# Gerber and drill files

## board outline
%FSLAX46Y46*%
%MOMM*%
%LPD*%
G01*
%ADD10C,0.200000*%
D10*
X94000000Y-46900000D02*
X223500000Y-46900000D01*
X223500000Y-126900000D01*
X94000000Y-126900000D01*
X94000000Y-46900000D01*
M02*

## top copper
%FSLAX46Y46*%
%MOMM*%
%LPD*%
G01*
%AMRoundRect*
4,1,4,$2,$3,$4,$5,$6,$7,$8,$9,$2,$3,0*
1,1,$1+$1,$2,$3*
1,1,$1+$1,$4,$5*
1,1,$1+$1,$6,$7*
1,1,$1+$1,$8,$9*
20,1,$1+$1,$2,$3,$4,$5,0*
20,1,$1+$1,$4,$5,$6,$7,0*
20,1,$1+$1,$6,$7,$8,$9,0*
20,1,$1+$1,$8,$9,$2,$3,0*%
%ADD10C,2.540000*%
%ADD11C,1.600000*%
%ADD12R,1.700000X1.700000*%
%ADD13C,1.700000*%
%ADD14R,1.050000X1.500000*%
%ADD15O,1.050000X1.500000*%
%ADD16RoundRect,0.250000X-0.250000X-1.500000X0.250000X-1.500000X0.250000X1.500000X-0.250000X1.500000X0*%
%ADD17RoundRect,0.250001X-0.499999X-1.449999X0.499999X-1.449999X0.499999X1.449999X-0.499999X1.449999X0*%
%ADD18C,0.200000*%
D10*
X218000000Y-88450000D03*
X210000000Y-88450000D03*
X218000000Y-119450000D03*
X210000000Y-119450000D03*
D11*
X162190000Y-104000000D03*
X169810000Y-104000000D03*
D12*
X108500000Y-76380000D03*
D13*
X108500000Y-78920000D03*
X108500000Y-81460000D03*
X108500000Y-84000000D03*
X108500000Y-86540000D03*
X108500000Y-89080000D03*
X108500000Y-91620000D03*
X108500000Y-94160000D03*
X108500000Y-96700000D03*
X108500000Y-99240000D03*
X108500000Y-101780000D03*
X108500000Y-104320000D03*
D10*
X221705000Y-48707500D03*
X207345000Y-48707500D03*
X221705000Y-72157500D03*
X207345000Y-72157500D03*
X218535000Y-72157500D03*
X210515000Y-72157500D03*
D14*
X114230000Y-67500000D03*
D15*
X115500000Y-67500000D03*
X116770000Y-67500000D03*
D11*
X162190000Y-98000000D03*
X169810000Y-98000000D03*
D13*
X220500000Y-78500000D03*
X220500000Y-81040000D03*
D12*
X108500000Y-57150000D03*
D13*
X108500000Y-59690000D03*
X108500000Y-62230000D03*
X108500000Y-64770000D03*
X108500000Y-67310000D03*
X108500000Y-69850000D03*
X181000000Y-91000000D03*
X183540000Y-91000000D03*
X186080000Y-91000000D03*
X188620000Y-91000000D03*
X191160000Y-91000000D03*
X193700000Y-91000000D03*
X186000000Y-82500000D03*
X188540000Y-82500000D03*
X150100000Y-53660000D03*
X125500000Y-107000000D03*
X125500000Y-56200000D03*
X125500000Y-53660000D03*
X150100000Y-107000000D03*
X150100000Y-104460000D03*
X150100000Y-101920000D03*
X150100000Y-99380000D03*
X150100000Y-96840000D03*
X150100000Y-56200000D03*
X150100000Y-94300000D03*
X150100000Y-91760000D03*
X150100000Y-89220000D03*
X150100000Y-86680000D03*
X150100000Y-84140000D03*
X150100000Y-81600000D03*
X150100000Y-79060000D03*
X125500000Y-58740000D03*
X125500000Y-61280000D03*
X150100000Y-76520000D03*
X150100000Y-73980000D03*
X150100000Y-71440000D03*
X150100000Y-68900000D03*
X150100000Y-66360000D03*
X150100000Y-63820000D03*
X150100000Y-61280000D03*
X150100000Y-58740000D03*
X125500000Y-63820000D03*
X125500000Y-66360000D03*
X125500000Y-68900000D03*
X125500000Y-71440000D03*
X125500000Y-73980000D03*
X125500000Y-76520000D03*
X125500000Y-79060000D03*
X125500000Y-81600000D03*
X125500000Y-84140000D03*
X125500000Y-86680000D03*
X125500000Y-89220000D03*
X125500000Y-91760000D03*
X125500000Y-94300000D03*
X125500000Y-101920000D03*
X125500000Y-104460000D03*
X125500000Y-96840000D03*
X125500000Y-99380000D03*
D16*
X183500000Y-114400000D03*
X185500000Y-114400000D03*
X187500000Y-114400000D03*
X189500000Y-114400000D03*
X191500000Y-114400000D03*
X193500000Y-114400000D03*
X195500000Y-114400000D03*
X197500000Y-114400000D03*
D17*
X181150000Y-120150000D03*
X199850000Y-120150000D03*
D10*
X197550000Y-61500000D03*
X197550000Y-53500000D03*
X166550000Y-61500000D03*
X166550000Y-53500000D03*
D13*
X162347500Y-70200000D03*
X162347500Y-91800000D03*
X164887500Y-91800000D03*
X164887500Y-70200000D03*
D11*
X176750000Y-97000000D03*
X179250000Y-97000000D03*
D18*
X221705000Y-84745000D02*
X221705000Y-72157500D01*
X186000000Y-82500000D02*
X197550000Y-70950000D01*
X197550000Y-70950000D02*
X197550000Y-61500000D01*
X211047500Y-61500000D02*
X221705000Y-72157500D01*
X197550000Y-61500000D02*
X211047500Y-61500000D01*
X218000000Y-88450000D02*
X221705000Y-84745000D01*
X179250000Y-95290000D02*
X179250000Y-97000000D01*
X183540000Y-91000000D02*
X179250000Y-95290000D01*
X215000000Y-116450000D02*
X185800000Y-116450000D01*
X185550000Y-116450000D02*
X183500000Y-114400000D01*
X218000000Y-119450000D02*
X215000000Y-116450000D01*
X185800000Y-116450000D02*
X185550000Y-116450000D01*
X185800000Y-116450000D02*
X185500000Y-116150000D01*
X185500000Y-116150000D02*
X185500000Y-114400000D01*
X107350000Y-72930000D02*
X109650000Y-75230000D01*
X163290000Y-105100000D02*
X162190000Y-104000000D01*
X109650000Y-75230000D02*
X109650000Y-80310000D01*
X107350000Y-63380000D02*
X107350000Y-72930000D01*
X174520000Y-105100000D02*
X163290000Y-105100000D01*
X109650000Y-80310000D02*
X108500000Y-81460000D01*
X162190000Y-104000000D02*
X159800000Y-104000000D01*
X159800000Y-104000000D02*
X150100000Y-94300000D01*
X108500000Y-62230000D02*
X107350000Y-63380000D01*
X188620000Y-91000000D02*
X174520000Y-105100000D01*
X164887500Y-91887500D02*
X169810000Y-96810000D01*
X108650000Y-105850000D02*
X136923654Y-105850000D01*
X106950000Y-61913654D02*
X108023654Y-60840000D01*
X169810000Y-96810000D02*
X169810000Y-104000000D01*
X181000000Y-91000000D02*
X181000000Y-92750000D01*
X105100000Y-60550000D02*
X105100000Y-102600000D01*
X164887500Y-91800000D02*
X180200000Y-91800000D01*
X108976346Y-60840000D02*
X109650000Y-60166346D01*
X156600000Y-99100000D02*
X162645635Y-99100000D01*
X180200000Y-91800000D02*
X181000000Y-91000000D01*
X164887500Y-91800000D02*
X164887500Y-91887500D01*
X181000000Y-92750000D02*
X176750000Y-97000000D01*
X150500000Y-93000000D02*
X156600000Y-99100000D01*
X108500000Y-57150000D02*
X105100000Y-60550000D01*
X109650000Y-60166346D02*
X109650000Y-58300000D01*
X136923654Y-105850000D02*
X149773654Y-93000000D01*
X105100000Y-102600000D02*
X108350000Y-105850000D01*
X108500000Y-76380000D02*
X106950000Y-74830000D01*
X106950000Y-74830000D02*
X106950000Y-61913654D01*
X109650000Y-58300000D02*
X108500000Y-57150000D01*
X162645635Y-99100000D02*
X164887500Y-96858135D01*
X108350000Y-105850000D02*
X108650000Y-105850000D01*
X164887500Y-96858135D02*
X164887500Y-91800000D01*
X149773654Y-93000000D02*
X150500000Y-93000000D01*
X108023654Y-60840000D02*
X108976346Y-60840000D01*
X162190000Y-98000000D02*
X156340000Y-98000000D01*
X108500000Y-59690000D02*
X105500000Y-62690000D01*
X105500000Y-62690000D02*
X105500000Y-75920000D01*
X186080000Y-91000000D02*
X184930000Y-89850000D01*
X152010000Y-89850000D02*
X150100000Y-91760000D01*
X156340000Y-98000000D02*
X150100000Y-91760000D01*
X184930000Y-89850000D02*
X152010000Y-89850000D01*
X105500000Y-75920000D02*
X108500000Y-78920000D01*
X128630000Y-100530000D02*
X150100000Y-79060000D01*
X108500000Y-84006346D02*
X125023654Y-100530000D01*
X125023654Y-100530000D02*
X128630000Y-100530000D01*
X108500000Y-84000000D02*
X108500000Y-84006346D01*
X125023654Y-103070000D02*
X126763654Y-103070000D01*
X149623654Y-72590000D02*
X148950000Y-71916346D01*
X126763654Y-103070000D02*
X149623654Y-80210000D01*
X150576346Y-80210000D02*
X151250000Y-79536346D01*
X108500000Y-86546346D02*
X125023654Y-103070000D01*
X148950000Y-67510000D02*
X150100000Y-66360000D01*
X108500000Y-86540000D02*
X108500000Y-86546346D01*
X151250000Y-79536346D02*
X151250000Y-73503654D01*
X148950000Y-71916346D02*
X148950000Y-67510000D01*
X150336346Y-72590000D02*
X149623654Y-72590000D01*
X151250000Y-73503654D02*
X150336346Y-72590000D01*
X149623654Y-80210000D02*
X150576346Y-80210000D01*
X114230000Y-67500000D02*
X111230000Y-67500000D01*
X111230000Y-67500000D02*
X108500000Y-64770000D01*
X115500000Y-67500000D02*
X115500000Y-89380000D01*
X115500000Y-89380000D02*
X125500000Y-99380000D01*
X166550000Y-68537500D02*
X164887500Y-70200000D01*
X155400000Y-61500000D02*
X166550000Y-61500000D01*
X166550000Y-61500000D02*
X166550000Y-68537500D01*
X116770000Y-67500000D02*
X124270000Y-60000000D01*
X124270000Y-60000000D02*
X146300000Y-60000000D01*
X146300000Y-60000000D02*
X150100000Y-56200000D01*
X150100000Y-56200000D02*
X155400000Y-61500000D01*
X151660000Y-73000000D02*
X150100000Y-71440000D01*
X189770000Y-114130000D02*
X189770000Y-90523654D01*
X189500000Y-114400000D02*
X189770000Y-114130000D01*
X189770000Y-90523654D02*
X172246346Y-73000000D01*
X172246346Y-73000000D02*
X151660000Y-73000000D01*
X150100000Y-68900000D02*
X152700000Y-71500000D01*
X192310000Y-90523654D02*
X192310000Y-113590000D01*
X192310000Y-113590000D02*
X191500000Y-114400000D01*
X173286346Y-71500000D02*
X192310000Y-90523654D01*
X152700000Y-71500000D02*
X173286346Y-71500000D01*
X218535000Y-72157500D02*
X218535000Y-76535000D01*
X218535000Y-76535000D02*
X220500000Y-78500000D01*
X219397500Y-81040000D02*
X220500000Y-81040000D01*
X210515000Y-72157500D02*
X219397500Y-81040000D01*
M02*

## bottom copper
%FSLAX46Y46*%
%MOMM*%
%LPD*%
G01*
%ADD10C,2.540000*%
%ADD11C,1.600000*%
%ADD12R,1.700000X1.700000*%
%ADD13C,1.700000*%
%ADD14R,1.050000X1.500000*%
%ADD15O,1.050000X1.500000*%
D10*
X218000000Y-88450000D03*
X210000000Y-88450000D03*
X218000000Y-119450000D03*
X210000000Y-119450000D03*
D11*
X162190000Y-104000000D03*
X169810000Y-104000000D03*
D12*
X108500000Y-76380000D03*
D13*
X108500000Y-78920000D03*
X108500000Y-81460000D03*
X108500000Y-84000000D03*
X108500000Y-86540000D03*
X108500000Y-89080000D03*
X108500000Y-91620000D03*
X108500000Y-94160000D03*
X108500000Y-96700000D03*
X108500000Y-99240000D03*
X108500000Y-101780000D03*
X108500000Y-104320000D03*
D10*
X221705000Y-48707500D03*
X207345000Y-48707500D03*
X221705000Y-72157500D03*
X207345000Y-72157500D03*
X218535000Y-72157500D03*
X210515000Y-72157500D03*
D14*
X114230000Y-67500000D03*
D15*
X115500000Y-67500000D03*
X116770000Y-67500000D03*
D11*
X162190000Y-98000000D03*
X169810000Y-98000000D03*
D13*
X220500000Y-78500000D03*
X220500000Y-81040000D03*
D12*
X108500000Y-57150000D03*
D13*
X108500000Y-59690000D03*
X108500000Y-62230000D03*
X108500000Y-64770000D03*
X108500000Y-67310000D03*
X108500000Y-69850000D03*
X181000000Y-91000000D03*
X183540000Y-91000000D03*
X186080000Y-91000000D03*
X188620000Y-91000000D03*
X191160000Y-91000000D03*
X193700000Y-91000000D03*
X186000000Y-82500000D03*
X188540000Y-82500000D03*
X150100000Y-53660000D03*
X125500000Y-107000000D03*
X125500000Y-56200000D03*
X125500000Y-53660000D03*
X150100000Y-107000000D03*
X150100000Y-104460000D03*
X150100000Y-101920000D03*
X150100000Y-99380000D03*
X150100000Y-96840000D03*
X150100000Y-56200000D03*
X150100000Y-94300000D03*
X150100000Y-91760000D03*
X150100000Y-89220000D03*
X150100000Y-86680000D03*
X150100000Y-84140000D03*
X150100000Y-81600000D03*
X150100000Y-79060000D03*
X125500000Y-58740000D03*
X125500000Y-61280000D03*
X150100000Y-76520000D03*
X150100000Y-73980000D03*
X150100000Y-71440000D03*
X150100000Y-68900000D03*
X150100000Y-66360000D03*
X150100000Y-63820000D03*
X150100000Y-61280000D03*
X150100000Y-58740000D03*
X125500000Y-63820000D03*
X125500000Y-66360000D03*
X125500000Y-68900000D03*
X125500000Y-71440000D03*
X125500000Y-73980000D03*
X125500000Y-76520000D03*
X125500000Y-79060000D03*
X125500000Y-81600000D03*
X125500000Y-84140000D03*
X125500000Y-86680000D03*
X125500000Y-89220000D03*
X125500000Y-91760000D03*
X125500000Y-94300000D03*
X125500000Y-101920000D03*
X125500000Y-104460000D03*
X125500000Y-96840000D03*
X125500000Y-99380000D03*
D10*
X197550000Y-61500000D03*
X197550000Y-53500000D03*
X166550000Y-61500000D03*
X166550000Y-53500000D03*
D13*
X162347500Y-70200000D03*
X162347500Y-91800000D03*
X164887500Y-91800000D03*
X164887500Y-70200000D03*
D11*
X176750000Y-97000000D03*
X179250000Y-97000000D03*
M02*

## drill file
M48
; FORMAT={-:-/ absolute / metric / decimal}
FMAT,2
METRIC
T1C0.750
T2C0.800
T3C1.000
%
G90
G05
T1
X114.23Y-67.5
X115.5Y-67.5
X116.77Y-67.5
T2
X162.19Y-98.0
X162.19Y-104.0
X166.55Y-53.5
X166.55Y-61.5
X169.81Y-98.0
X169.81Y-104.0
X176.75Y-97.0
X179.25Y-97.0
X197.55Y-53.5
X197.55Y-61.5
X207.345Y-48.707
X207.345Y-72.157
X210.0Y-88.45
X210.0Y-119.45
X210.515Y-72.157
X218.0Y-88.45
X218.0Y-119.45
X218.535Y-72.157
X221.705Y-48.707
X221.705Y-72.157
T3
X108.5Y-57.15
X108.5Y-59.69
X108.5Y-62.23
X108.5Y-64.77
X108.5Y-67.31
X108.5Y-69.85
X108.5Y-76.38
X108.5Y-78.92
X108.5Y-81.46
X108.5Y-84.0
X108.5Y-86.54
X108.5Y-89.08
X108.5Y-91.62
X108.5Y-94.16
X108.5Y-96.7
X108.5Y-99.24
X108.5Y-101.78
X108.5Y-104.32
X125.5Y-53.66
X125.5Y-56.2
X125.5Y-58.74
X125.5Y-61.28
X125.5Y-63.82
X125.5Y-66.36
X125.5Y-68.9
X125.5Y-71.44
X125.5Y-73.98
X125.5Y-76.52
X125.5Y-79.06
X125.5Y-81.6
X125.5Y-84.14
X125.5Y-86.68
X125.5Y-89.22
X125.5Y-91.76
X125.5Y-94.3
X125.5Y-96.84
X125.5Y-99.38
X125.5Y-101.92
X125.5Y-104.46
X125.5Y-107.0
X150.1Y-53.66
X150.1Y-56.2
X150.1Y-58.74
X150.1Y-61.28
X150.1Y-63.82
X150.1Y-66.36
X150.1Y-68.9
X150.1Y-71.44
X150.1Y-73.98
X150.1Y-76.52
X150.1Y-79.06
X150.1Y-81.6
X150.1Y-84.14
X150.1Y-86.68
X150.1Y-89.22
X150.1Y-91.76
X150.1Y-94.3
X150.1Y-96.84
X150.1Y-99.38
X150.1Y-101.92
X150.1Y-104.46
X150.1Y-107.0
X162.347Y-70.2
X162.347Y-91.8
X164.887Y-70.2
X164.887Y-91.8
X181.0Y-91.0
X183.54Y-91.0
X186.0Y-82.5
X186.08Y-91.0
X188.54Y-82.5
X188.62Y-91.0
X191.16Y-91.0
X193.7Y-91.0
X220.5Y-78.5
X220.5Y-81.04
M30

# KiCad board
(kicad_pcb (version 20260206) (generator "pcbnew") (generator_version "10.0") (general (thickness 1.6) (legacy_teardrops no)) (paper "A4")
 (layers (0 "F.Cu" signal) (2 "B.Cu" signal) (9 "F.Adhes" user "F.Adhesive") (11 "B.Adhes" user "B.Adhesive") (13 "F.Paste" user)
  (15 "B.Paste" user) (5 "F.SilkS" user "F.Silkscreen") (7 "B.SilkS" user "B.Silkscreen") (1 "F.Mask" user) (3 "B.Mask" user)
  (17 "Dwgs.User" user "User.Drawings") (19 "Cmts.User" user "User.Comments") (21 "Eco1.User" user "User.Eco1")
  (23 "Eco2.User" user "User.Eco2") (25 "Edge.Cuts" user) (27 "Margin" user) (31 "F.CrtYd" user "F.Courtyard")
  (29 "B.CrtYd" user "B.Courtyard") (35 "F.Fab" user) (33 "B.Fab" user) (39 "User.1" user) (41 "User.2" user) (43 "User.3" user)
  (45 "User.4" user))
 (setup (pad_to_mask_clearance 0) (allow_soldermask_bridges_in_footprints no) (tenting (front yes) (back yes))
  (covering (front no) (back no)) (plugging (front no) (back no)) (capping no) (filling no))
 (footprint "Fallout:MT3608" (layer "F.Cu") (at 222.5 85.95 -90)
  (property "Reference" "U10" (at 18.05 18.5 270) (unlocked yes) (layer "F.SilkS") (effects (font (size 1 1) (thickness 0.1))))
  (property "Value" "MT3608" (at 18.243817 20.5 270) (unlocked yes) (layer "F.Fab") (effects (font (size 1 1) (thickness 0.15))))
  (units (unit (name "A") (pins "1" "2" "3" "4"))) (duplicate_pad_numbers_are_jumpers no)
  (pad "1" thru_hole circle (at 2.5 4.5 270) (size 2.54 2.54) (drill 0.8) (layers "*.Cu" "*.Mask") (remove_unused_layers no)
   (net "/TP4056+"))
  (pad "2" thru_hole circle (at 2.5 12.5 270) (size 2.54 2.54) (drill 0.8) (layers "*.Cu" "*.Mask") (remove_unused_layers no) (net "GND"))
  (pad "3" thru_hole circle (at 33.5 4.5 270) (size 2.54 2.54) (drill 0.8) (layers "*.Cu" "*.Mask") (remove_unused_layers no) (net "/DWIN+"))
  (pad "4" thru_hole circle (at 33.5 12.5 270) (size 2.54 2.54) (drill 0.8) (layers "*.Cu" "*.Mask") (remove_unused_layers no) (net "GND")))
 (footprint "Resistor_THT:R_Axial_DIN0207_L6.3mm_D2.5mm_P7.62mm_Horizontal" (layer "F.Cu") (at 162.19 104)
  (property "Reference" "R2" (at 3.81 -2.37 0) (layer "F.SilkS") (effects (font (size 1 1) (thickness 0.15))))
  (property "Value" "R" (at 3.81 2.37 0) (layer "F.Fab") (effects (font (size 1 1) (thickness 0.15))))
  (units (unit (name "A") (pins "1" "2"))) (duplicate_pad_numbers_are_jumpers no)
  (pad "1" thru_hole circle (at 0 0) (size 1.6 1.6) (drill 0.8) (layers "*.Cu" "*.Mask") (remove_unused_layers no) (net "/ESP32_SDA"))
  (pad "2" thru_hole circle (at 7.62 0) (size 1.6 1.6) (drill 0.8) (layers "*.Cu" "*.Mask") (remove_unused_layers no) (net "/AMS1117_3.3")))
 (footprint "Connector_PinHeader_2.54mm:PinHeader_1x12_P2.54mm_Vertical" (layer "F.Cu") (at 108.5 76.38)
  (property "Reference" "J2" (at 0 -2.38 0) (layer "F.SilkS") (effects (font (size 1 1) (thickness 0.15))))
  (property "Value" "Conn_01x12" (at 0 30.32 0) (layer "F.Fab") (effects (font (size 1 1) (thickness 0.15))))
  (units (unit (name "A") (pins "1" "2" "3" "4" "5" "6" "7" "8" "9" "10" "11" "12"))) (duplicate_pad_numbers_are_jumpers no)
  (pad "1" thru_hole rect (at 0 0) (size 1.7 1.7) (drill 1) (layers "*.Cu" "*.Mask") (remove_unused_layers no) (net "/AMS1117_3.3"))
  (pad "2" thru_hole circle (at 0 2.54) (size 1.7 1.7) (drill 1) (layers "*.Cu" "*.Mask") (remove_unused_layers no) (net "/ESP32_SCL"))
  (pad "3" thru_hole circle (at 0 5.08) (size 1.7 1.7) (drill 1) (layers "*.Cu" "*.Mask") (remove_unused_layers no) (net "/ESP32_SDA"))
  (pad "4" thru_hole circle (at 0 7.62) (size 1.7 1.7) (drill 1) (layers "*.Cu" "*.Mask") (remove_unused_layers no) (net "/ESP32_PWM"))
  (pad "5" thru_hole circle (at 0 10.16) (size 1.7 1.7) (drill 1) (layers "*.Cu" "*.Mask") (remove_unused_layers no) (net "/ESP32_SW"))
  (pad "6" thru_hole circle (at 0 12.7) (size 1.7 1.7) (drill 1) (layers "*.Cu" "*.Mask") (remove_unused_layers no)
   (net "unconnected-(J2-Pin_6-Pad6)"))
  (pad "7" thru_hole circle (at 0 15.24) (size 1.7 1.7) (drill 1) (layers "*.Cu" "*.Mask") (remove_unused_layers no)
   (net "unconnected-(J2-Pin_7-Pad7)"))
  (pad "8" thru_hole circle (at 0 17.78) (size 1.7 1.7) (drill 1) (layers "*.Cu" "*.Mask") (remove_unused_layers no)
   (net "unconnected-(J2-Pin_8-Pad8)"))
  (pad "9" thru_hole circle (at 0 20.32) (size 1.7 1.7) (drill 1) (layers "*.Cu" "*.Mask") (remove_unused_layers no)
   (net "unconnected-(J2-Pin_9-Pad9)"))
  (pad "10" thru_hole circle (at 0 22.86) (size 1.7 1.7) (drill 1) (layers "*.Cu" "*.Mask") (remove_unused_layers no)
   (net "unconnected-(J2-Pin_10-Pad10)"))
  (pad "11" thru_hole circle (at 0 25.4) (size 1.7 1.7) (drill 1) (layers "*.Cu" "*.Mask") (remove_unused_layers no)
   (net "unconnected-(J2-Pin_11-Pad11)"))
  (pad "12" thru_hole circle (at 0 27.94) (size 1.7 1.7) (drill 1) (layers "*.Cu" "*.Mask") (remove_unused_layers no)
   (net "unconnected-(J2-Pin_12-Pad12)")))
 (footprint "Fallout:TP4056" (layer "F.Cu") (at 223.1 47.3125 -90)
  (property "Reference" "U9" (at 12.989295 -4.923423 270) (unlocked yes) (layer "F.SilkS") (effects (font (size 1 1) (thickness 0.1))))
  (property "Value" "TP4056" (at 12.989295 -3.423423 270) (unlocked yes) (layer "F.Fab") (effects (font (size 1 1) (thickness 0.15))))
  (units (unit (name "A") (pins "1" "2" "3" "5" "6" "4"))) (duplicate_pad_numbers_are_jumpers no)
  (pad "1" thru_hole circle (at 1.395 1.395 270) (size 2.54 2.54) (drill 0.8) (layers "*.Cu" "*.Mask") (remove_unused_layers no)
   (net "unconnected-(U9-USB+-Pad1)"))
  (pad "2" thru_hole circle (at 1.395 15.755 270) (size 2.54 2.54) (drill 0.8) (layers "*.Cu" "*.Mask") (remove_unused_layers no)
   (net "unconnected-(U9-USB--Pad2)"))
  (pad "3" thru_hole circle (at 24.845 1.395 270) (size 2.54 2.54) (drill 0.8) (layers "*.Cu" "*.Mask") (remove_unused_layers no)
   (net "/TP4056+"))
  (pad "4" thru_hole circle (at 24.845 15.755 270) (size 2.54 2.54) (drill 0.8) (layers "*.Cu" "*.Mask") (remove_unused_layers no)
   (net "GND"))
  (pad "5" thru_hole circle (at 24.845 4.565 270) (size 2.54 2.54) (drill 0.8) (layers "*.Cu" "*.Mask") (remove_unused_layers no)
   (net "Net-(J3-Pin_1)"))
  (pad "6" thru_hole circle (at 24.845 12.585 270) (size 2.54 2.54) (drill 0.8) (layers "*.Cu" "*.Mask") (remove_unused_layers no)
   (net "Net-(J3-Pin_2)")))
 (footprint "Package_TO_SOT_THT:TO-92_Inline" (layer "F.Cu") (at 114.23 67.5)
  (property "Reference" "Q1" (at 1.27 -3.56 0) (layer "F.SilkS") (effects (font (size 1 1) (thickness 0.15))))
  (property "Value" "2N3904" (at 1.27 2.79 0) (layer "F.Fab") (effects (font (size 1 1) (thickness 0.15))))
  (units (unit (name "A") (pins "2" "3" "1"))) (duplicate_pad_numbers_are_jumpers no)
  (pad "1" thru_hole rect (at 0 0) (size 1.05 1.5) (drill 0.75) (layers "*.Cu" "*.Mask") (remove_unused_layers no) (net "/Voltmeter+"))
  (pad "2" thru_hole oval (at 1.27 0) (size 1.05 1.5) (drill 0.75) (layers "*.Cu" "*.Mask") (remove_unused_layers no) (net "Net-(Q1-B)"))
  (pad "3" thru_hole oval (at 2.54 0) (size 1.05 1.5) (drill 0.75) (layers "*.Cu" "*.Mask") (remove_unused_layers no) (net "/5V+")))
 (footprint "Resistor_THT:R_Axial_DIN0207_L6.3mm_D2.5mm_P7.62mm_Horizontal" (layer "F.Cu") (at 162.19 98)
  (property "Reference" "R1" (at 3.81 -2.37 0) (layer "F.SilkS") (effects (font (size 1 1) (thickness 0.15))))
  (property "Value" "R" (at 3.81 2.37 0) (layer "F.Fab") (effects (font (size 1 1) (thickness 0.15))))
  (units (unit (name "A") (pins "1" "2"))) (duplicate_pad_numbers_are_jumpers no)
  (pad "1" thru_hole circle (at 0 0) (size 1.6 1.6) (drill 0.8) (layers "*.Cu" "*.Mask") (remove_unused_layers no) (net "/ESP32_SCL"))
  (pad "2" thru_hole circle (at 7.62 0) (size 1.6 1.6) (drill 0.8) (layers "*.Cu" "*.Mask") (remove_unused_layers no) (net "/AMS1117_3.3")))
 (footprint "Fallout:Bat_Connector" (layer "F.Cu") (at 227.2 79.84 -90)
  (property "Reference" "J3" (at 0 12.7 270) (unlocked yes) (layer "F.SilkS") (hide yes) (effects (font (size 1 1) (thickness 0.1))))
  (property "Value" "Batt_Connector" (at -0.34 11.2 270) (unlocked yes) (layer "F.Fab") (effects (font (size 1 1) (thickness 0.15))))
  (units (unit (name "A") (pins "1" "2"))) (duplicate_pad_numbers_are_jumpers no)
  (pad "1" thru_hole circle (at -1.34 6.7 270) (size 1.7 1.7) (drill 1) (layers "*.Cu" "*.Mask") (remove_unused_layers no)
   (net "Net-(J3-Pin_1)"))
  (pad "2" thru_hole circle (at 1.2 6.7 270) (size 1.7 1.7) (drill 1) (layers "*.Cu" "*.Mask") (remove_unused_layers no)
   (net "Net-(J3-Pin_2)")))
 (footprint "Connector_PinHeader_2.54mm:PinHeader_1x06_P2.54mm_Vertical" (layer "F.Cu") (at 108.5 57.15)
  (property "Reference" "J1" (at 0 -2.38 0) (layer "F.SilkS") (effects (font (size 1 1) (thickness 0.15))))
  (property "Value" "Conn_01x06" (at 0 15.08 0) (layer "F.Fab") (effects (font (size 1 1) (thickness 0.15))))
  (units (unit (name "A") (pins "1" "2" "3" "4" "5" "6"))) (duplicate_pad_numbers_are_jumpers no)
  (pad "1" thru_hole rect (at 0 0) (size 1.7 1.7) (drill 1) (layers "*.Cu" "*.Mask") (remove_unused_layers no) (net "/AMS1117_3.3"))
  (pad "2" thru_hole circle (at 0 2.54) (size 1.7 1.7) (drill 1) (layers "*.Cu" "*.Mask") (remove_unused_layers no) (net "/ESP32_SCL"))
  (pad "3" thru_hole circle (at 0 5.08) (size 1.7 1.7) (drill 1) (layers "*.Cu" "*.Mask") (remove_unused_layers no) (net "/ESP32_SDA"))
  (pad "4" thru_hole circle (at 0 7.62) (size 1.7 1.7) (drill 1) (layers "*.Cu" "*.Mask") (remove_unused_layers no) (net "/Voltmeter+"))
  (pad "5" thru_hole circle (at 0 10.16) (size 1.7 1.7) (drill 1) (layers "*.Cu" "*.Mask") (remove_unused_layers no) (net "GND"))
  (pad "6" thru_hole circle (at 0 12.7) (size 1.7 1.7) (drill 1) (layers "*.Cu" "*.Mask") (remove_unused_layers no)
   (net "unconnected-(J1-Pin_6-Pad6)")))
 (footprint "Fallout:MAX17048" (layer "F.Cu") (at 187.190406 68.664095)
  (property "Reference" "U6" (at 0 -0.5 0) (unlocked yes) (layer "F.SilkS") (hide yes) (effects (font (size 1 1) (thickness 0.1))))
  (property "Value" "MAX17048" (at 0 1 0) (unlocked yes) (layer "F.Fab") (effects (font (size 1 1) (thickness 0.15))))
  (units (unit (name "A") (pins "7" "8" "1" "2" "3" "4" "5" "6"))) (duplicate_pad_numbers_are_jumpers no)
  (pad "1" thru_hole circle (at -6.190406 22.335905) (size 1.7 1.7) (drill 1) (layers "*.Cu" "*.Mask") (remove_unused_layers no)
   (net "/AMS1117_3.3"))
  (pad "2" thru_hole circle (at -3.650406 22.335905) (size 1.7 1.7) (drill 1) (layers "*.Cu" "*.Mask") (remove_unused_layers no) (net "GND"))
  (pad "3" thru_hole circle (at -1.110406 22.335905) (size 1.7 1.7) (drill 1) (layers "*.Cu" "*.Mask") (remove_unused_layers no)
   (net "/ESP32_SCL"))
  (pad "4" thru_hole circle (at 1.429594 22.335905) (size 1.7 1.7) (drill 1) (layers "*.Cu" "*.Mask") (remove_unused_layers no)
   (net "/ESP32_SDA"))
  (pad "5" thru_hole circle (at 3.969594 22.335905) (size 1.7 1.7) (drill 1) (layers "*.Cu" "*.Mask") (remove_unused_layers no)
   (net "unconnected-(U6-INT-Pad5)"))
  (pad "6" thru_hole circle (at 6.509594 22.335905) (size 1.7 1.7) (drill 1) (layers "*.Cu" "*.Mask") (remove_unused_layers no)
   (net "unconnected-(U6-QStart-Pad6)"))
  (pad "7" thru_hole circle (at -1.190406 13.835905) (size 1.7 1.7) (drill 1) (layers "*.Cu" "*.Mask") (remove_unused_layers no)
   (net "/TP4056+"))
  (pad "8" thru_hole circle (at 1.349594 13.835905) (size 1.7 1.7) (drill 1) (layers "*.Cu" "*.Mask") (remove_unused_layers no) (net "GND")))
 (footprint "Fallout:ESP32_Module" (layer "F.Cu") (at 137.843597 134.499017 180)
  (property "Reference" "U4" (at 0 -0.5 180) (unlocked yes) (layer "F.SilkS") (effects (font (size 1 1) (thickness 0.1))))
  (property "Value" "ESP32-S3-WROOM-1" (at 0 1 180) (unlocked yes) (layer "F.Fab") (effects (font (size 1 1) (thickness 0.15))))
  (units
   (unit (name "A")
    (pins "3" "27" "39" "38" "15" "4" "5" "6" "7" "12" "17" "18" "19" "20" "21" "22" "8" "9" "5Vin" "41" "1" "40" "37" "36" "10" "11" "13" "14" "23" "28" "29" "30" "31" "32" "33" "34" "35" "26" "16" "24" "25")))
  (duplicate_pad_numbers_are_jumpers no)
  (pad "1" thru_hole circle (at -12.256403 80.839017 180) (size 1.7 1.7) (drill 1) (layers "*.Cu" "*.Mask") (remove_unused_layers no)
   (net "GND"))
  (pad "1" thru_hole circle (at 12.343597 27.499017 180) (size 1.7 1.7) (drill 1) (layers "*.Cu" "*.Mask") (remove_unused_layers no)
   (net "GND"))
  (pad "1" thru_hole circle (at 12.343597 78.299017 180) (size 1.7 1.7) (drill 1) (layers "*.Cu" "*.Mask") (remove_unused_layers no)
   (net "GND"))
  (pad "1" thru_hole circle (at 12.343597 80.839017 180) (size 1.7 1.7) (drill 1) (layers "*.Cu" "*.Mask") (remove_unused_layers no)
   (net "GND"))
  (pad "2" thru_hole circle (at -12.256403 27.499017 180) (size 1.7 1.7) (drill 1) (layers "*.Cu" "*.Mask") (remove_unused_layers no))
  (pad "2" thru_hole circle (at -12.256403 30.039017 180) (size 1.7 1.7) (drill 1) (layers "*.Cu" "*.Mask") (remove_unused_layers no))
  (pad "3" thru_hole circle (at -12.256403 32.579017 180) (size 1.7 1.7) (drill 1) (layers "*.Cu" "*.Mask") (remove_unused_layers no)
   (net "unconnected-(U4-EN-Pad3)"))
  (pad "4" thru_hole circle (at -12.256403 35.119017 180) (size 1.7 1.7) (drill 1) (layers "*.Cu" "*.Mask") (remove_unused_layers no)
   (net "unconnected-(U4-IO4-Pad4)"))
  (pad "5" thru_hole circle (at -12.256403 37.659017 180) (size 1.7 1.7) (drill 1) (layers "*.Cu" "*.Mask") (remove_unused_layers no)
   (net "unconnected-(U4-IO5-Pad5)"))
  (pad "5Vin" thru_hole circle (at -12.256403 78.299017 180) (size 1.7 1.7) (drill 1) (layers "*.Cu" "*.Mask") (remove_unused_layers no)
   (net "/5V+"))
  (pad "6" thru_hole circle (at -12.256403 40.199017 180) (size 1.7 1.7) (drill 1) (layers "*.Cu" "*.Mask") (remove_unused_layers no)
   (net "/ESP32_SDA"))
  (pad "7" thru_hole circle (at -12.256403 42.739017 180) (size 1.7 1.7) (drill 1) (layers "*.Cu" "*.Mask") (remove_unused_layers no)
   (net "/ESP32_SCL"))
  (pad "8" thru_hole circle (at -12.256403 45.279017 180) (size 1.7 1.7) (drill 1) (layers "*.Cu" "*.Mask") (remove_unused_layers no)
   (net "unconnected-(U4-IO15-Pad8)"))
  (pad "9" thru_hole circle (at -12.256403 47.819017 180) (size 1.7 1.7) (drill 1) (layers "*.Cu" "*.Mask") (remove_unused_layers no)
   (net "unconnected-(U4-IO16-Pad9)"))
  (pad "10" thru_hole circle (at -12.256403 50.359017 180) (size 1.7 1.7) (drill 1) (layers "*.Cu" "*.Mask") (remove_unused_layers no)
   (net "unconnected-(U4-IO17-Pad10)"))
  (pad "11" thru_hole circle (at -12.256403 52.899017 180) (size 1.7 1.7) (drill 1) (layers "*.Cu" "*.Mask") (remove_unused_layers no)
   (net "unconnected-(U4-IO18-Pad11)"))
  (pad "12" thru_hole circle (at -12.256403 55.439017 180) (size 1.7 1.7) (drill 1) (layers "*.Cu" "*.Mask") (remove_unused_layers no)
   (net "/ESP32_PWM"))
  (pad "13" thru_hole circle (at 12.343597 75.759017 180) (size 1.7 1.7) (drill 1) (layers "*.Cu" "*.Mask") (remove_unused_layers no)
   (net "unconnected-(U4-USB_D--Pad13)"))
  (pad "14" thru_hole circle (at 12.343597 73.219017 180) (size 1.7 1.7) (drill 1) (layers "*.Cu" "*.Mask") (remove_unused_layers no)
   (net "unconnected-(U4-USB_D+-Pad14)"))
  (pad "15" thru_hole circle (at -12.256403 57.979017 180) (size 1.7 1.7) (drill 1) (layers "*.Cu" "*.Mask") (remove_unused_layers no)
   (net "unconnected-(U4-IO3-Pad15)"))
  (pad "16" thru_hole circle (at -12.256403 60.519017 180) (size 1.7 1.7) (drill 1) (layers "*.Cu" "*.Mask") (remove_unused_layers no)
   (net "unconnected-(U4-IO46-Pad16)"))
  (pad "17" thru_hole circle (at -12.256403 63.059017 180) (size 1.7 1.7) (drill 1) (layers "*.Cu" "*.Mask") (remove_unused_layers no)
   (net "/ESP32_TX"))
  (pad "18" thru_hole circle (at -12.256403 65.599017 180) (size 1.7 1.7) (drill 1) (layers "*.Cu" "*.Mask") (remove_unused_layers no)
   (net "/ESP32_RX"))
  (pad "19" thru_hole circle (at -12.256403 68.139017 180) (size 1.7 1.7) (drill 1) (layers "*.Cu" "*.Mask") (remove_unused_layers no)
   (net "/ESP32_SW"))
  (pad "20" thru_hole circle (at -12.256403 70.679017 180) (size 1.7 1.7) (drill 1) (layers "*.Cu" "*.Mask") (remove_unused_layers no)
   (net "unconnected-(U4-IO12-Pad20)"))
  (pad "21" thru_hole circle (at -12.256403 73.219017 180) (size 1.7 1.7) (drill 1) (layers "*.Cu" "*.Mask") (remove_unused_layers no)
   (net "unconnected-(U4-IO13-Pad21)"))
  (pad "22" thru_hole circle (at -12.256403 75.759017 180) (size 1.7 1.7) (drill 1) (layers "*.Cu" "*.Mask") (remove_unused_layers no)
   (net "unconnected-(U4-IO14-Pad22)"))
  (pad "23" thru_hole circle (at 12.343597 70.679017 180) (size 1.7 1.7) (drill 1) (layers "*.Cu" "*.Mask") (remove_unused_layers no)
   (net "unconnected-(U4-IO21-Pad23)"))
  (pad "24" thru_hole circle (at 12.343597 68.139017 180) (size 1.7 1.7) (drill 1) (layers "*.Cu" "*.Mask") (remove_unused_layers no)
   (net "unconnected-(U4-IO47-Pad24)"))
  (pad "25" thru_hole circle (at 12.343597 65.599017 180) (size 1.7 1.7) (drill 1) (layers "*.Cu" "*.Mask") (remove_unused_layers no)
   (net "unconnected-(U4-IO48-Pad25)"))
  (pad "26" thru_hole circle (at 12.343597 63.059017 180) (size 1.7 1.7) (drill 1) (layers "*.Cu" "*.Mask") (remove_unused_layers no)
   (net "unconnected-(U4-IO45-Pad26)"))
  (pad "27" thru_hole circle (at 12.343597 60.519017 180) (size 1.7 1.7) (drill 1) (layers "*.Cu" "*.Mask") (remove_unused_layers no)
   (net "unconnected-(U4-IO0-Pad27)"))
  (pad "28" thru_hole circle (at 12.343597 57.979017 180) (size 1.7 1.7) (drill 1) (layers "*.Cu" "*.Mask") (remove_unused_layers no)
   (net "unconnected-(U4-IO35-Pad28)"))
  (pad "29" thru_hole circle (at 12.343597 55.439017 180) (size 1.7 1.7) (drill 1) (layers "*.Cu" "*.Mask") (remove_unused_layers no)
   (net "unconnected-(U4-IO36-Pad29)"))
  (pad "30" thru_hole circle (at 12.343597 52.899017 180) (size 1.7 1.7) (drill 1) (layers "*.Cu" "*.Mask") (remove_unused_layers no)
   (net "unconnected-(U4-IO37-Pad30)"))
  (pad "31" thru_hole circle (at 12.343597 50.359017 180) (size 1.7 1.7) (drill 1) (layers "*.Cu" "*.Mask") (remove_unused_layers no)
   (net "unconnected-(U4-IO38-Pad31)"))
  (pad "32" thru_hole circle (at 12.343597 47.819017 180) (size 1.7 1.7) (drill 1) (layers "*.Cu" "*.Mask") (remove_unused_layers no)
   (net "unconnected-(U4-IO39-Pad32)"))
  (pad "33" thru_hole circle (at 12.343597 45.279017 180) (size 1.7 1.7) (drill 1) (layers "*.Cu" "*.Mask") (remove_unused_layers no)
   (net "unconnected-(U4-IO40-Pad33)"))
  (pad "34" thru_hole circle (at 12.343597 42.739017 180) (size 1.7 1.7) (drill 1) (layers "*.Cu" "*.Mask") (remove_unused_layers no)
   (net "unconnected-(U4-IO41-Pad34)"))
  (pad "35" thru_hole circle (at 12.343597 40.199017 180) (size 1.7 1.7) (drill 1) (layers "*.Cu" "*.Mask") (remove_unused_layers no)
   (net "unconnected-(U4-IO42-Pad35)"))
  (pad "36" thru_hole circle (at 12.343597 32.579017 180) (size 1.7 1.7) (drill 1) (layers "*.Cu" "*.Mask") (remove_unused_layers no)
   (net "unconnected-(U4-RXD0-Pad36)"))
  (pad "37" thru_hole circle (at 12.343597 30.039017 180) (size 1.7 1.7) (drill 1) (layers "*.Cu" "*.Mask") (remove_unused_layers no)
   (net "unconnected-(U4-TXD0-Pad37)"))
  (pad "38" thru_hole circle (at 12.343597 37.659017 180) (size 1.7 1.7) (drill 1) (layers "*.Cu" "*.Mask") (remove_unused_layers no)
   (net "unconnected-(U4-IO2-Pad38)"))
  (pad "39" thru_hole circle (at 12.343597 35.119017 180) (size 1.7 1.7) (drill 1) (layers "*.Cu" "*.Mask") (remove_unused_layers no)
   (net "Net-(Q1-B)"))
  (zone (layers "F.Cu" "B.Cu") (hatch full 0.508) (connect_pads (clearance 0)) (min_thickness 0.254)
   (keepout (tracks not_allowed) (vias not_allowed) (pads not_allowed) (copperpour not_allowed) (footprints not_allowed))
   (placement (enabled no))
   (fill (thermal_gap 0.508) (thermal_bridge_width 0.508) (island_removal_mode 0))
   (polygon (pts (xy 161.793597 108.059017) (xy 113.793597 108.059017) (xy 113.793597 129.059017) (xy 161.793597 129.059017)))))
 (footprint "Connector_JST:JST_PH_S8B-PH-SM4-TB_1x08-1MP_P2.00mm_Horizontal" (layer "F.Cu") (at 190.5 117.25)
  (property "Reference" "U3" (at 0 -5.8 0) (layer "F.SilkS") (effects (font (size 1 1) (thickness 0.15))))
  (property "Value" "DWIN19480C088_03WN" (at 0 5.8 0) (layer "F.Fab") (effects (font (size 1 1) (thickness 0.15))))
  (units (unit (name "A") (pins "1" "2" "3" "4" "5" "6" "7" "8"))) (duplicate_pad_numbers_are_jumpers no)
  (pad "1" smd roundrect (at -7 -2.85) (size 1 3.5) (layers "F.Cu" "F.Mask" "F.Paste") (roundrect_rratio 0.25) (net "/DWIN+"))
  (pad "2" smd roundrect (at -5 -2.85) (size 1 3.5) (layers "F.Cu" "F.Mask" "F.Paste") (roundrect_rratio 0.25) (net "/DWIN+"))
  (pad "3" smd roundrect (at -3 -2.85) (size 1 3.5) (layers "F.Cu" "F.Mask" "F.Paste") (roundrect_rratio 0.25)
   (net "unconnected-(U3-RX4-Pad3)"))
  (pad "4" smd roundrect (at -1 -2.85) (size 1 3.5) (layers "F.Cu" "F.Mask" "F.Paste") (roundrect_rratio 0.25) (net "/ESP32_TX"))
  (pad "5" smd roundrect (at 1 -2.85) (size 1 3.5) (layers "F.Cu" "F.Mask" "F.Paste") (roundrect_rratio 0.25) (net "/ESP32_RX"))
  (pad "6" smd roundrect (at 3 -2.85) (size 1 3.5) (layers "F.Cu" "F.Mask" "F.Paste") (roundrect_rratio 0.25)
   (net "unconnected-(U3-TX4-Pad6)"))
  (pad "7" smd roundrect (at 5 -2.85) (size 1 3.5) (layers "F.Cu" "F.Mask" "F.Paste") (roundrect_rratio 0.25)
   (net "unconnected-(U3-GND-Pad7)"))
  (pad "8" smd roundrect (at 7 -2.85) (size 1 3.5) (layers "F.Cu" "F.Mask" "F.Paste") (roundrect_rratio 0.25) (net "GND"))
  (pad "MP" smd roundrect (at -9.35 2.9) (size 1.5 3.4) (layers "F.Cu" "F.Mask" "F.Paste") (roundrect_rratio 0.166667))
  (pad "MP" smd roundrect (at 9.35 2.9) (size 1.5 3.4) (layers "F.Cu" "F.Mask" "F.Paste") (roundrect_rratio 0.166667)))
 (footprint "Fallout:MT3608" (layer "F.Cu") (at 200.05 66 180)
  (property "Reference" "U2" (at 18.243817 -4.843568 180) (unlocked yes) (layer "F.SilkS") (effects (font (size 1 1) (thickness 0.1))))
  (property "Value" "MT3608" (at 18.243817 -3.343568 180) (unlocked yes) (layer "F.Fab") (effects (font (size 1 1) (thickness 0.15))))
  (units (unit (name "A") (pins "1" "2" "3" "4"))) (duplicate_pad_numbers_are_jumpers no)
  (pad "1" thru_hole circle (at 2.5 4.5 180) (size 2.54 2.54) (drill 0.8) (layers "*.Cu" "*.Mask") (remove_unused_layers no)
   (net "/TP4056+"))
  (pad "2" thru_hole circle (at 2.5 12.5 180) (size 2.54 2.54) (drill 0.8) (layers "*.Cu" "*.Mask") (remove_unused_layers no) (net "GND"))
  (pad "3" thru_hole circle (at 33.5 4.5 180) (size 2.54 2.54) (drill 0.8) (layers "*.Cu" "*.Mask") (remove_unused_layers no) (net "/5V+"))
  (pad "4" thru_hole circle (at 33.5 12.5 180) (size 2.54 2.54) (drill 0.8) (layers "*.Cu" "*.Mask") (remove_unused_layers no) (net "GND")))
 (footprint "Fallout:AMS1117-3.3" (layer "F.Cu") (at 172.9875 80.2 -90)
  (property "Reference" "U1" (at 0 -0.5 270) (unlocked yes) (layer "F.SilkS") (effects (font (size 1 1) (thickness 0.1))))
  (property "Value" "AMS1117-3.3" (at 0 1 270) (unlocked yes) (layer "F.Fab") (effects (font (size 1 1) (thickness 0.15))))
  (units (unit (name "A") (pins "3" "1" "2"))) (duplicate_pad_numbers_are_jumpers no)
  (pad "1" thru_hole circle (at -10 10.64 270) (size 1.7 1.7) (drill 1) (layers "*.Cu" "*.Mask") (remove_unused_layers no) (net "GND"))
  (pad "1" thru_hole circle (at 11.6 10.64 270) (size 1.7 1.7) (drill 1) (layers "*.Cu" "*.Mask") (remove_unused_layers no) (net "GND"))
  (pad "2" thru_hole circle (at 11.6 8.1 270) (size 1.7 1.7) (drill 1) (layers "*.Cu" "*.Mask") (remove_unused_layers no)
   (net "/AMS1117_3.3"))
  (pad "3" thru_hole circle (at -10 8.1 270) (size 1.7 1.7) (drill 1) (layers "*.Cu" "*.Mask") (remove_unused_layers no) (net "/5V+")))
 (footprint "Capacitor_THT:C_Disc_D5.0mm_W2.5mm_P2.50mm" (layer "F.Cu") (at 176.75 97)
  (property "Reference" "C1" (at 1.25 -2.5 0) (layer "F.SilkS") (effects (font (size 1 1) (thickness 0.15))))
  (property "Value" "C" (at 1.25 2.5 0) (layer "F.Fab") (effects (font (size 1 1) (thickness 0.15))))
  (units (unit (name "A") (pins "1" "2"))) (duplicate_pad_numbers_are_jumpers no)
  (pad "1" thru_hole circle (at 0 0) (size 1.6 1.6) (drill 0.8) (layers "*.Cu" "*.Mask") (remove_unused_layers no) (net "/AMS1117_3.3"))
  (pad "2" thru_hole circle (at 2.5 0) (size 1.6 1.6) (drill 0.8) (layers "*.Cu" "*.Mask") (remove_unused_layers no) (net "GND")))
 (gr_rect (start 94 46.9) (end 223.5 126.9) (stroke (width 0.2) (type solid)) (fill no) (layer "Edge.Cuts"))
 (segment (start 221.705 84.745) (end 221.705 72.1575) (width 0.2) (layer "F.Cu") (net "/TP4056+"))
 (segment (start 186 82.5) (end 197.55 70.95) (width 0.2) (layer "F.Cu") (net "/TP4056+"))
 (segment (start 197.55 70.95) (end 197.55 61.5) (width 0.2) (layer "F.Cu") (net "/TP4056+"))
 (segment (start 211.0475 61.5) (end 221.705 72.1575) (width 0.2) (layer "F.Cu") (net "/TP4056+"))
 (segment (start 197.55 61.5) (end 211.0475 61.5) (width 0.2) (layer "F.Cu") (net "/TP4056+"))
 (segment (start 218 88.45) (end 221.705 84.745) (width 0.2) (layer "F.Cu") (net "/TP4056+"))
 (segment (start 179.25 95.29) (end 179.25 97) (width 0.2) (layer "F.Cu") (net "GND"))
 (segment (start 183.54 91) (end 179.25 95.29) (width 0.2) (layer "F.Cu") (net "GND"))
 (segment (start 215 116.45) (end 185.8 116.45) (width 0.2) (layer "F.Cu") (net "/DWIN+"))
 (segment (start 185.55 116.45) (end 183.5 114.4) (width 0.2) (layer "F.Cu") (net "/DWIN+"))
 (segment (start 218 119.45) (end 215 116.45) (width 0.2) (layer "F.Cu") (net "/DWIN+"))
 (segment (start 185.8 116.45) (end 185.55 116.45) (width 0.2) (layer "F.Cu") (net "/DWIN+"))
 (segment (start 185.8 116.45) (end 185.5 116.15) (width 0.2) (layer "F.Cu") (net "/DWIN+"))
 (segment (start 185.5 116.15) (end 185.5 114.4) (width 0.2) (layer "F.Cu") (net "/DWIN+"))
 (segment (start 107.35 72.93) (end 109.65 75.23) (width 0.2) (layer "F.Cu") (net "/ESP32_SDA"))
 (segment (start 163.29 105.1) (end 162.19 104) (width 0.2) (layer "F.Cu") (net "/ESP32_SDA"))
 (segment (start 109.65 75.23) (end 109.65 80.31) (width 0.2) (layer "F.Cu") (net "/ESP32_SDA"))
 (segment (start 107.35 63.38) (end 107.35 72.93) (width 0.2) (layer "F.Cu") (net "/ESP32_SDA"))
 (segment (start 174.52 105.1) (end 163.29 105.1) (width 0.2) (layer "F.Cu") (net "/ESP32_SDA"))
 (segment (start 109.65 80.31) (end 108.5 81.46) (width 0.2) (layer "F.Cu") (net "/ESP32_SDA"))
 (segment (start 162.19 104) (end 159.8 104) (width 0.2) (layer "F.Cu") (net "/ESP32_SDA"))
 (segment (start 159.8 104) (end 150.1 94.3) (width 0.2) (layer "F.Cu") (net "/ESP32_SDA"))
 (segment (start 108.5 62.23) (end 107.35 63.38) (width 0.2) (layer "F.Cu") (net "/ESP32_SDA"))
 (segment (start 188.62 91) (end 174.52 105.1) (width 0.2) (layer "F.Cu") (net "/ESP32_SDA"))
 (segment (start 164.8875 91.8875) (end 169.81 96.81) (width 0.2) (layer "F.Cu") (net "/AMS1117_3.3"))
 (segment (start 108.65 105.85) (end 136.923654 105.85) (width 0.2) (layer "F.Cu") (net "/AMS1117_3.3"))
 (segment (start 106.95 61.913654) (end 108.023654 60.84) (width 0.2) (layer "F.Cu") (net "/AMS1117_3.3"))
 (segment (start 169.81 96.81) (end 169.81 104) (width 0.2) (layer "F.Cu") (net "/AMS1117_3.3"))
 (segment (start 181 91) (end 181 92.75) (width 0.2) (layer "F.Cu") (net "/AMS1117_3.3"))
 (segment (start 105.1 60.55) (end 105.1 102.6) (width 0.2) (layer "F.Cu") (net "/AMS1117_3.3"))
 (segment (start 164.8875 91.8) (end 180.2 91.8) (width 0.2) (layer "F.Cu") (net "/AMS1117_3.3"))
 (segment (start 108.976346 60.84) (end 109.65 60.166346) (width 0.2) (layer "F.Cu") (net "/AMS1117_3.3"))
 (segment (start 156.6 99.1) (end 162.645635 99.1) (width 0.2) (layer "F.Cu") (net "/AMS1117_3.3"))
 (segment (start 180.2 91.8) (end 181 91) (width 0.2) (layer "F.Cu") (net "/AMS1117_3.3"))
 (segment (start 164.8875 91.8) (end 164.8875 91.8875) (width 0.2) (layer "F.Cu") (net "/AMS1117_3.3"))
 (segment (start 181 92.75) (end 176.75 97) (width 0.2) (layer "F.Cu") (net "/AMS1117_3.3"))
 (segment (start 150.5 93) (end 156.6 99.1) (width 0.2) (layer "F.Cu") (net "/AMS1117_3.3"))
 (segment (start 108.5 57.15) (end 105.1 60.55) (width 0.2) (layer "F.Cu") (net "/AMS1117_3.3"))
 (segment (start 109.65 60.166346) (end 109.65 58.3) (width 0.2) (layer "F.Cu") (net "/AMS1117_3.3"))
 (segment (start 136.923654 105.85) (end 149.773654 93) (width 0.2) (layer "F.Cu") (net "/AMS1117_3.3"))
 (segment (start 105.1 102.6) (end 108.35 105.85) (width 0.2) (layer "F.Cu") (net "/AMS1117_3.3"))
 (segment (start 108.5 76.38) (end 106.95 74.83) (width 0.2) (layer "F.Cu") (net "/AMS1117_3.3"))
 (segment (start 106.95 74.83) (end 106.95 61.913654) (width 0.2) (layer "F.Cu") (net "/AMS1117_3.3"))
 (segment (start 109.65 58.3) (end 108.5 57.15) (width 0.2) (layer "F.Cu") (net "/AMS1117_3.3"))
 (segment (start 162.645635 99.1) (end 164.8875 96.858135) (width 0.2) (layer "F.Cu") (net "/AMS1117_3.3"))
 (segment (start 108.35 105.85) (end 108.65 105.85) (width 0.2) (layer "F.Cu") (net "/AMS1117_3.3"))
 (segment (start 164.8875 96.858135) (end 164.8875 91.8) (width 0.2) (layer "F.Cu") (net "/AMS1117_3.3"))
 (segment (start 149.773654 93) (end 150.5 93) (width 0.2) (layer "F.Cu") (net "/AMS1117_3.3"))
 (segment (start 108.023654 60.84) (end 108.976346 60.84) (width 0.2) (layer "F.Cu") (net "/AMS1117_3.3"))
 (segment (start 162.19 98) (end 156.34 98) (width 0.2) (layer "F.Cu") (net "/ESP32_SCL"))
 (segment (start 108.5 59.69) (end 105.5 62.69) (width 0.2) (layer "F.Cu") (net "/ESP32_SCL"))
 (segment (start 105.5 62.69) (end 105.5 75.92) (width 0.2) (layer "F.Cu") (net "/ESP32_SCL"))
 (segment (start 186.08 91) (end 184.93 89.85) (width 0.2) (layer "F.Cu") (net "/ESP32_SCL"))
 (segment (start 152.01 89.85) (end 150.1 91.76) (width 0.2) (layer "F.Cu") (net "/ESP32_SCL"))
 (segment (start 156.34 98) (end 150.1 91.76) (width 0.2) (layer "F.Cu") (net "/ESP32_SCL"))
 (segment (start 184.93 89.85) (end 152.01 89.85) (width 0.2) (layer "F.Cu") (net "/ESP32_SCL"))
 (segment (start 105.5 75.92) (end 108.5 78.92) (width 0.2) (layer "F.Cu") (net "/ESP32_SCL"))
 (segment (start 128.63 100.53) (end 150.1 79.06) (width 0.2) (layer "F.Cu") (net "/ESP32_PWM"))
 (segment (start 108.5 84.006346) (end 125.023654 100.53) (width 0.2) (layer "F.Cu") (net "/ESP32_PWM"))
 (segment (start 125.023654 100.53) (end 128.63 100.53) (width 0.2) (layer "F.Cu") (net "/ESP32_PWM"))
 (segment (start 108.5 84) (end 108.5 84.006346) (width 0.2) (layer "F.Cu") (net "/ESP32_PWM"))
 (segment (start 125.023654 103.07) (end 126.763654 103.07) (width 0.2) (layer "F.Cu") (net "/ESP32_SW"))
 (segment (start 149.623654 72.59) (end 148.95 71.916346) (width 0.2) (layer "F.Cu") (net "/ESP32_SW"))
 (segment (start 126.763654 103.07) (end 149.623654 80.21) (width 0.2) (layer "F.Cu") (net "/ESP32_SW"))
 (segment (start 150.576346 80.21) (end 151.25 79.536346) (width 0.2) (layer "F.Cu") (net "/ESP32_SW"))
 (segment (start 108.5 86.546346) (end 125.023654 103.07) (width 0.2) (layer "F.Cu") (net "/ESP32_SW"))
 (segment (start 148.95 67.51) (end 150.1 66.36) (width 0.2) (layer "F.Cu") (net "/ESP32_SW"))
 (segment (start 108.5 86.54) (end 108.5 86.546346) (width 0.2) (layer "F.Cu") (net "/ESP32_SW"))
 (segment (start 151.25 79.536346) (end 151.25 73.503654) (width 0.2) (layer "F.Cu") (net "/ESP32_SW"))
 (segment (start 148.95 71.916346) (end 148.95 67.51) (width 0.2) (layer "F.Cu") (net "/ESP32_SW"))
 (segment (start 150.336346 72.59) (end 149.623654 72.59) (width 0.2) (layer "F.Cu") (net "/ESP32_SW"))
 (segment (start 151.25 73.503654) (end 150.336346 72.59) (width 0.2) (layer "F.Cu") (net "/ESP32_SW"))
 (segment (start 149.623654 80.21) (end 150.576346 80.21) (width 0.2) (layer "F.Cu") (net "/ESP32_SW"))
 (segment (start 114.23 67.5) (end 111.23 67.5) (width 0.2) (layer "F.Cu") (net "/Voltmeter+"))
 (segment (start 111.23 67.5) (end 108.5 64.77) (width 0.2) (layer "F.Cu") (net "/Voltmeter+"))
 (segment (start 115.5 67.5) (end 115.5 89.38) (width 0.2) (layer "F.Cu") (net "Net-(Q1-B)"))
 (segment (start 115.5 89.38) (end 125.5 99.38) (width 0.2) (layer "F.Cu") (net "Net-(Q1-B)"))
 (segment (start 166.55 68.5375) (end 164.8875 70.2) (width 0.2) (layer "F.Cu") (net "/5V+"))
 (segment (start 155.4 61.5) (end 166.55 61.5) (width 0.2) (layer "F.Cu") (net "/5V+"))
 (segment (start 166.55 61.5) (end 166.55 68.5375) (width 0.2) (layer "F.Cu") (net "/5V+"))
 (segment (start 116.77 67.5) (end 124.27 60) (width 0.2) (layer "F.Cu") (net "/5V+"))
 (segment (start 124.27 60) (end 146.3 60) (width 0.2) (layer "F.Cu") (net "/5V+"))
 (segment (start 146.3 60) (end 150.1 56.2) (width 0.2) (layer "F.Cu") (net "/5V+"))
 (segment (start 150.1 56.2) (end 155.4 61.5) (width 0.2) (layer "F.Cu") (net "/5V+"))
 (segment (start 151.66 73) (end 150.1 71.44) (width 0.2) (layer "F.Cu") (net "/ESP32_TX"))
 (segment (start 189.77 114.13) (end 189.77 90.523654) (width 0.2) (layer "F.Cu") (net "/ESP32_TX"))
 (segment (start 189.5 114.4) (end 189.77 114.13) (width 0.2) (layer "F.Cu") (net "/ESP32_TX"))
 (segment (start 189.77 90.523654) (end 172.246346 73) (width 0.2) (layer "F.Cu") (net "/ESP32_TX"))
 (segment (start 172.246346 73) (end 151.66 73) (width 0.2) (layer "F.Cu") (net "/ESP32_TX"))
 (segment (start 150.1 68.9) (end 152.7 71.5) (width 0.2) (layer "F.Cu") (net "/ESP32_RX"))
 (segment (start 192.31 90.523654) (end 192.31 113.59) (width 0.2) (layer "F.Cu") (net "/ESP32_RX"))
 (segment (start 192.31 113.59) (end 191.5 114.4) (width 0.2) (layer "F.Cu") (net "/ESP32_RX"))
 (segment (start 173.286346 71.5) (end 192.31 90.523654) (width 0.2) (layer "F.Cu") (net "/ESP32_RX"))
 (segment (start 152.7 71.5) (end 173.286346 71.5) (width 0.2) (layer "F.Cu") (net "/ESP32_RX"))
 (segment (start 218.535 72.1575) (end 218.535 76.535) (width 0.2) (layer "F.Cu") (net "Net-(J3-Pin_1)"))
 (segment (start 218.535 76.535) (end 220.5 78.5) (width 0.2) (layer "F.Cu") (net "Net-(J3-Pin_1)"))
 (segment (start 219.3975 81.04) (end 220.5 81.04) (width 0.2) (layer "F.Cu") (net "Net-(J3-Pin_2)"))
 (segment (start 210.515 72.1575) (end 219.3975 81.04) (width 0.2) (layer "F.Cu") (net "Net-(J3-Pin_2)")))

